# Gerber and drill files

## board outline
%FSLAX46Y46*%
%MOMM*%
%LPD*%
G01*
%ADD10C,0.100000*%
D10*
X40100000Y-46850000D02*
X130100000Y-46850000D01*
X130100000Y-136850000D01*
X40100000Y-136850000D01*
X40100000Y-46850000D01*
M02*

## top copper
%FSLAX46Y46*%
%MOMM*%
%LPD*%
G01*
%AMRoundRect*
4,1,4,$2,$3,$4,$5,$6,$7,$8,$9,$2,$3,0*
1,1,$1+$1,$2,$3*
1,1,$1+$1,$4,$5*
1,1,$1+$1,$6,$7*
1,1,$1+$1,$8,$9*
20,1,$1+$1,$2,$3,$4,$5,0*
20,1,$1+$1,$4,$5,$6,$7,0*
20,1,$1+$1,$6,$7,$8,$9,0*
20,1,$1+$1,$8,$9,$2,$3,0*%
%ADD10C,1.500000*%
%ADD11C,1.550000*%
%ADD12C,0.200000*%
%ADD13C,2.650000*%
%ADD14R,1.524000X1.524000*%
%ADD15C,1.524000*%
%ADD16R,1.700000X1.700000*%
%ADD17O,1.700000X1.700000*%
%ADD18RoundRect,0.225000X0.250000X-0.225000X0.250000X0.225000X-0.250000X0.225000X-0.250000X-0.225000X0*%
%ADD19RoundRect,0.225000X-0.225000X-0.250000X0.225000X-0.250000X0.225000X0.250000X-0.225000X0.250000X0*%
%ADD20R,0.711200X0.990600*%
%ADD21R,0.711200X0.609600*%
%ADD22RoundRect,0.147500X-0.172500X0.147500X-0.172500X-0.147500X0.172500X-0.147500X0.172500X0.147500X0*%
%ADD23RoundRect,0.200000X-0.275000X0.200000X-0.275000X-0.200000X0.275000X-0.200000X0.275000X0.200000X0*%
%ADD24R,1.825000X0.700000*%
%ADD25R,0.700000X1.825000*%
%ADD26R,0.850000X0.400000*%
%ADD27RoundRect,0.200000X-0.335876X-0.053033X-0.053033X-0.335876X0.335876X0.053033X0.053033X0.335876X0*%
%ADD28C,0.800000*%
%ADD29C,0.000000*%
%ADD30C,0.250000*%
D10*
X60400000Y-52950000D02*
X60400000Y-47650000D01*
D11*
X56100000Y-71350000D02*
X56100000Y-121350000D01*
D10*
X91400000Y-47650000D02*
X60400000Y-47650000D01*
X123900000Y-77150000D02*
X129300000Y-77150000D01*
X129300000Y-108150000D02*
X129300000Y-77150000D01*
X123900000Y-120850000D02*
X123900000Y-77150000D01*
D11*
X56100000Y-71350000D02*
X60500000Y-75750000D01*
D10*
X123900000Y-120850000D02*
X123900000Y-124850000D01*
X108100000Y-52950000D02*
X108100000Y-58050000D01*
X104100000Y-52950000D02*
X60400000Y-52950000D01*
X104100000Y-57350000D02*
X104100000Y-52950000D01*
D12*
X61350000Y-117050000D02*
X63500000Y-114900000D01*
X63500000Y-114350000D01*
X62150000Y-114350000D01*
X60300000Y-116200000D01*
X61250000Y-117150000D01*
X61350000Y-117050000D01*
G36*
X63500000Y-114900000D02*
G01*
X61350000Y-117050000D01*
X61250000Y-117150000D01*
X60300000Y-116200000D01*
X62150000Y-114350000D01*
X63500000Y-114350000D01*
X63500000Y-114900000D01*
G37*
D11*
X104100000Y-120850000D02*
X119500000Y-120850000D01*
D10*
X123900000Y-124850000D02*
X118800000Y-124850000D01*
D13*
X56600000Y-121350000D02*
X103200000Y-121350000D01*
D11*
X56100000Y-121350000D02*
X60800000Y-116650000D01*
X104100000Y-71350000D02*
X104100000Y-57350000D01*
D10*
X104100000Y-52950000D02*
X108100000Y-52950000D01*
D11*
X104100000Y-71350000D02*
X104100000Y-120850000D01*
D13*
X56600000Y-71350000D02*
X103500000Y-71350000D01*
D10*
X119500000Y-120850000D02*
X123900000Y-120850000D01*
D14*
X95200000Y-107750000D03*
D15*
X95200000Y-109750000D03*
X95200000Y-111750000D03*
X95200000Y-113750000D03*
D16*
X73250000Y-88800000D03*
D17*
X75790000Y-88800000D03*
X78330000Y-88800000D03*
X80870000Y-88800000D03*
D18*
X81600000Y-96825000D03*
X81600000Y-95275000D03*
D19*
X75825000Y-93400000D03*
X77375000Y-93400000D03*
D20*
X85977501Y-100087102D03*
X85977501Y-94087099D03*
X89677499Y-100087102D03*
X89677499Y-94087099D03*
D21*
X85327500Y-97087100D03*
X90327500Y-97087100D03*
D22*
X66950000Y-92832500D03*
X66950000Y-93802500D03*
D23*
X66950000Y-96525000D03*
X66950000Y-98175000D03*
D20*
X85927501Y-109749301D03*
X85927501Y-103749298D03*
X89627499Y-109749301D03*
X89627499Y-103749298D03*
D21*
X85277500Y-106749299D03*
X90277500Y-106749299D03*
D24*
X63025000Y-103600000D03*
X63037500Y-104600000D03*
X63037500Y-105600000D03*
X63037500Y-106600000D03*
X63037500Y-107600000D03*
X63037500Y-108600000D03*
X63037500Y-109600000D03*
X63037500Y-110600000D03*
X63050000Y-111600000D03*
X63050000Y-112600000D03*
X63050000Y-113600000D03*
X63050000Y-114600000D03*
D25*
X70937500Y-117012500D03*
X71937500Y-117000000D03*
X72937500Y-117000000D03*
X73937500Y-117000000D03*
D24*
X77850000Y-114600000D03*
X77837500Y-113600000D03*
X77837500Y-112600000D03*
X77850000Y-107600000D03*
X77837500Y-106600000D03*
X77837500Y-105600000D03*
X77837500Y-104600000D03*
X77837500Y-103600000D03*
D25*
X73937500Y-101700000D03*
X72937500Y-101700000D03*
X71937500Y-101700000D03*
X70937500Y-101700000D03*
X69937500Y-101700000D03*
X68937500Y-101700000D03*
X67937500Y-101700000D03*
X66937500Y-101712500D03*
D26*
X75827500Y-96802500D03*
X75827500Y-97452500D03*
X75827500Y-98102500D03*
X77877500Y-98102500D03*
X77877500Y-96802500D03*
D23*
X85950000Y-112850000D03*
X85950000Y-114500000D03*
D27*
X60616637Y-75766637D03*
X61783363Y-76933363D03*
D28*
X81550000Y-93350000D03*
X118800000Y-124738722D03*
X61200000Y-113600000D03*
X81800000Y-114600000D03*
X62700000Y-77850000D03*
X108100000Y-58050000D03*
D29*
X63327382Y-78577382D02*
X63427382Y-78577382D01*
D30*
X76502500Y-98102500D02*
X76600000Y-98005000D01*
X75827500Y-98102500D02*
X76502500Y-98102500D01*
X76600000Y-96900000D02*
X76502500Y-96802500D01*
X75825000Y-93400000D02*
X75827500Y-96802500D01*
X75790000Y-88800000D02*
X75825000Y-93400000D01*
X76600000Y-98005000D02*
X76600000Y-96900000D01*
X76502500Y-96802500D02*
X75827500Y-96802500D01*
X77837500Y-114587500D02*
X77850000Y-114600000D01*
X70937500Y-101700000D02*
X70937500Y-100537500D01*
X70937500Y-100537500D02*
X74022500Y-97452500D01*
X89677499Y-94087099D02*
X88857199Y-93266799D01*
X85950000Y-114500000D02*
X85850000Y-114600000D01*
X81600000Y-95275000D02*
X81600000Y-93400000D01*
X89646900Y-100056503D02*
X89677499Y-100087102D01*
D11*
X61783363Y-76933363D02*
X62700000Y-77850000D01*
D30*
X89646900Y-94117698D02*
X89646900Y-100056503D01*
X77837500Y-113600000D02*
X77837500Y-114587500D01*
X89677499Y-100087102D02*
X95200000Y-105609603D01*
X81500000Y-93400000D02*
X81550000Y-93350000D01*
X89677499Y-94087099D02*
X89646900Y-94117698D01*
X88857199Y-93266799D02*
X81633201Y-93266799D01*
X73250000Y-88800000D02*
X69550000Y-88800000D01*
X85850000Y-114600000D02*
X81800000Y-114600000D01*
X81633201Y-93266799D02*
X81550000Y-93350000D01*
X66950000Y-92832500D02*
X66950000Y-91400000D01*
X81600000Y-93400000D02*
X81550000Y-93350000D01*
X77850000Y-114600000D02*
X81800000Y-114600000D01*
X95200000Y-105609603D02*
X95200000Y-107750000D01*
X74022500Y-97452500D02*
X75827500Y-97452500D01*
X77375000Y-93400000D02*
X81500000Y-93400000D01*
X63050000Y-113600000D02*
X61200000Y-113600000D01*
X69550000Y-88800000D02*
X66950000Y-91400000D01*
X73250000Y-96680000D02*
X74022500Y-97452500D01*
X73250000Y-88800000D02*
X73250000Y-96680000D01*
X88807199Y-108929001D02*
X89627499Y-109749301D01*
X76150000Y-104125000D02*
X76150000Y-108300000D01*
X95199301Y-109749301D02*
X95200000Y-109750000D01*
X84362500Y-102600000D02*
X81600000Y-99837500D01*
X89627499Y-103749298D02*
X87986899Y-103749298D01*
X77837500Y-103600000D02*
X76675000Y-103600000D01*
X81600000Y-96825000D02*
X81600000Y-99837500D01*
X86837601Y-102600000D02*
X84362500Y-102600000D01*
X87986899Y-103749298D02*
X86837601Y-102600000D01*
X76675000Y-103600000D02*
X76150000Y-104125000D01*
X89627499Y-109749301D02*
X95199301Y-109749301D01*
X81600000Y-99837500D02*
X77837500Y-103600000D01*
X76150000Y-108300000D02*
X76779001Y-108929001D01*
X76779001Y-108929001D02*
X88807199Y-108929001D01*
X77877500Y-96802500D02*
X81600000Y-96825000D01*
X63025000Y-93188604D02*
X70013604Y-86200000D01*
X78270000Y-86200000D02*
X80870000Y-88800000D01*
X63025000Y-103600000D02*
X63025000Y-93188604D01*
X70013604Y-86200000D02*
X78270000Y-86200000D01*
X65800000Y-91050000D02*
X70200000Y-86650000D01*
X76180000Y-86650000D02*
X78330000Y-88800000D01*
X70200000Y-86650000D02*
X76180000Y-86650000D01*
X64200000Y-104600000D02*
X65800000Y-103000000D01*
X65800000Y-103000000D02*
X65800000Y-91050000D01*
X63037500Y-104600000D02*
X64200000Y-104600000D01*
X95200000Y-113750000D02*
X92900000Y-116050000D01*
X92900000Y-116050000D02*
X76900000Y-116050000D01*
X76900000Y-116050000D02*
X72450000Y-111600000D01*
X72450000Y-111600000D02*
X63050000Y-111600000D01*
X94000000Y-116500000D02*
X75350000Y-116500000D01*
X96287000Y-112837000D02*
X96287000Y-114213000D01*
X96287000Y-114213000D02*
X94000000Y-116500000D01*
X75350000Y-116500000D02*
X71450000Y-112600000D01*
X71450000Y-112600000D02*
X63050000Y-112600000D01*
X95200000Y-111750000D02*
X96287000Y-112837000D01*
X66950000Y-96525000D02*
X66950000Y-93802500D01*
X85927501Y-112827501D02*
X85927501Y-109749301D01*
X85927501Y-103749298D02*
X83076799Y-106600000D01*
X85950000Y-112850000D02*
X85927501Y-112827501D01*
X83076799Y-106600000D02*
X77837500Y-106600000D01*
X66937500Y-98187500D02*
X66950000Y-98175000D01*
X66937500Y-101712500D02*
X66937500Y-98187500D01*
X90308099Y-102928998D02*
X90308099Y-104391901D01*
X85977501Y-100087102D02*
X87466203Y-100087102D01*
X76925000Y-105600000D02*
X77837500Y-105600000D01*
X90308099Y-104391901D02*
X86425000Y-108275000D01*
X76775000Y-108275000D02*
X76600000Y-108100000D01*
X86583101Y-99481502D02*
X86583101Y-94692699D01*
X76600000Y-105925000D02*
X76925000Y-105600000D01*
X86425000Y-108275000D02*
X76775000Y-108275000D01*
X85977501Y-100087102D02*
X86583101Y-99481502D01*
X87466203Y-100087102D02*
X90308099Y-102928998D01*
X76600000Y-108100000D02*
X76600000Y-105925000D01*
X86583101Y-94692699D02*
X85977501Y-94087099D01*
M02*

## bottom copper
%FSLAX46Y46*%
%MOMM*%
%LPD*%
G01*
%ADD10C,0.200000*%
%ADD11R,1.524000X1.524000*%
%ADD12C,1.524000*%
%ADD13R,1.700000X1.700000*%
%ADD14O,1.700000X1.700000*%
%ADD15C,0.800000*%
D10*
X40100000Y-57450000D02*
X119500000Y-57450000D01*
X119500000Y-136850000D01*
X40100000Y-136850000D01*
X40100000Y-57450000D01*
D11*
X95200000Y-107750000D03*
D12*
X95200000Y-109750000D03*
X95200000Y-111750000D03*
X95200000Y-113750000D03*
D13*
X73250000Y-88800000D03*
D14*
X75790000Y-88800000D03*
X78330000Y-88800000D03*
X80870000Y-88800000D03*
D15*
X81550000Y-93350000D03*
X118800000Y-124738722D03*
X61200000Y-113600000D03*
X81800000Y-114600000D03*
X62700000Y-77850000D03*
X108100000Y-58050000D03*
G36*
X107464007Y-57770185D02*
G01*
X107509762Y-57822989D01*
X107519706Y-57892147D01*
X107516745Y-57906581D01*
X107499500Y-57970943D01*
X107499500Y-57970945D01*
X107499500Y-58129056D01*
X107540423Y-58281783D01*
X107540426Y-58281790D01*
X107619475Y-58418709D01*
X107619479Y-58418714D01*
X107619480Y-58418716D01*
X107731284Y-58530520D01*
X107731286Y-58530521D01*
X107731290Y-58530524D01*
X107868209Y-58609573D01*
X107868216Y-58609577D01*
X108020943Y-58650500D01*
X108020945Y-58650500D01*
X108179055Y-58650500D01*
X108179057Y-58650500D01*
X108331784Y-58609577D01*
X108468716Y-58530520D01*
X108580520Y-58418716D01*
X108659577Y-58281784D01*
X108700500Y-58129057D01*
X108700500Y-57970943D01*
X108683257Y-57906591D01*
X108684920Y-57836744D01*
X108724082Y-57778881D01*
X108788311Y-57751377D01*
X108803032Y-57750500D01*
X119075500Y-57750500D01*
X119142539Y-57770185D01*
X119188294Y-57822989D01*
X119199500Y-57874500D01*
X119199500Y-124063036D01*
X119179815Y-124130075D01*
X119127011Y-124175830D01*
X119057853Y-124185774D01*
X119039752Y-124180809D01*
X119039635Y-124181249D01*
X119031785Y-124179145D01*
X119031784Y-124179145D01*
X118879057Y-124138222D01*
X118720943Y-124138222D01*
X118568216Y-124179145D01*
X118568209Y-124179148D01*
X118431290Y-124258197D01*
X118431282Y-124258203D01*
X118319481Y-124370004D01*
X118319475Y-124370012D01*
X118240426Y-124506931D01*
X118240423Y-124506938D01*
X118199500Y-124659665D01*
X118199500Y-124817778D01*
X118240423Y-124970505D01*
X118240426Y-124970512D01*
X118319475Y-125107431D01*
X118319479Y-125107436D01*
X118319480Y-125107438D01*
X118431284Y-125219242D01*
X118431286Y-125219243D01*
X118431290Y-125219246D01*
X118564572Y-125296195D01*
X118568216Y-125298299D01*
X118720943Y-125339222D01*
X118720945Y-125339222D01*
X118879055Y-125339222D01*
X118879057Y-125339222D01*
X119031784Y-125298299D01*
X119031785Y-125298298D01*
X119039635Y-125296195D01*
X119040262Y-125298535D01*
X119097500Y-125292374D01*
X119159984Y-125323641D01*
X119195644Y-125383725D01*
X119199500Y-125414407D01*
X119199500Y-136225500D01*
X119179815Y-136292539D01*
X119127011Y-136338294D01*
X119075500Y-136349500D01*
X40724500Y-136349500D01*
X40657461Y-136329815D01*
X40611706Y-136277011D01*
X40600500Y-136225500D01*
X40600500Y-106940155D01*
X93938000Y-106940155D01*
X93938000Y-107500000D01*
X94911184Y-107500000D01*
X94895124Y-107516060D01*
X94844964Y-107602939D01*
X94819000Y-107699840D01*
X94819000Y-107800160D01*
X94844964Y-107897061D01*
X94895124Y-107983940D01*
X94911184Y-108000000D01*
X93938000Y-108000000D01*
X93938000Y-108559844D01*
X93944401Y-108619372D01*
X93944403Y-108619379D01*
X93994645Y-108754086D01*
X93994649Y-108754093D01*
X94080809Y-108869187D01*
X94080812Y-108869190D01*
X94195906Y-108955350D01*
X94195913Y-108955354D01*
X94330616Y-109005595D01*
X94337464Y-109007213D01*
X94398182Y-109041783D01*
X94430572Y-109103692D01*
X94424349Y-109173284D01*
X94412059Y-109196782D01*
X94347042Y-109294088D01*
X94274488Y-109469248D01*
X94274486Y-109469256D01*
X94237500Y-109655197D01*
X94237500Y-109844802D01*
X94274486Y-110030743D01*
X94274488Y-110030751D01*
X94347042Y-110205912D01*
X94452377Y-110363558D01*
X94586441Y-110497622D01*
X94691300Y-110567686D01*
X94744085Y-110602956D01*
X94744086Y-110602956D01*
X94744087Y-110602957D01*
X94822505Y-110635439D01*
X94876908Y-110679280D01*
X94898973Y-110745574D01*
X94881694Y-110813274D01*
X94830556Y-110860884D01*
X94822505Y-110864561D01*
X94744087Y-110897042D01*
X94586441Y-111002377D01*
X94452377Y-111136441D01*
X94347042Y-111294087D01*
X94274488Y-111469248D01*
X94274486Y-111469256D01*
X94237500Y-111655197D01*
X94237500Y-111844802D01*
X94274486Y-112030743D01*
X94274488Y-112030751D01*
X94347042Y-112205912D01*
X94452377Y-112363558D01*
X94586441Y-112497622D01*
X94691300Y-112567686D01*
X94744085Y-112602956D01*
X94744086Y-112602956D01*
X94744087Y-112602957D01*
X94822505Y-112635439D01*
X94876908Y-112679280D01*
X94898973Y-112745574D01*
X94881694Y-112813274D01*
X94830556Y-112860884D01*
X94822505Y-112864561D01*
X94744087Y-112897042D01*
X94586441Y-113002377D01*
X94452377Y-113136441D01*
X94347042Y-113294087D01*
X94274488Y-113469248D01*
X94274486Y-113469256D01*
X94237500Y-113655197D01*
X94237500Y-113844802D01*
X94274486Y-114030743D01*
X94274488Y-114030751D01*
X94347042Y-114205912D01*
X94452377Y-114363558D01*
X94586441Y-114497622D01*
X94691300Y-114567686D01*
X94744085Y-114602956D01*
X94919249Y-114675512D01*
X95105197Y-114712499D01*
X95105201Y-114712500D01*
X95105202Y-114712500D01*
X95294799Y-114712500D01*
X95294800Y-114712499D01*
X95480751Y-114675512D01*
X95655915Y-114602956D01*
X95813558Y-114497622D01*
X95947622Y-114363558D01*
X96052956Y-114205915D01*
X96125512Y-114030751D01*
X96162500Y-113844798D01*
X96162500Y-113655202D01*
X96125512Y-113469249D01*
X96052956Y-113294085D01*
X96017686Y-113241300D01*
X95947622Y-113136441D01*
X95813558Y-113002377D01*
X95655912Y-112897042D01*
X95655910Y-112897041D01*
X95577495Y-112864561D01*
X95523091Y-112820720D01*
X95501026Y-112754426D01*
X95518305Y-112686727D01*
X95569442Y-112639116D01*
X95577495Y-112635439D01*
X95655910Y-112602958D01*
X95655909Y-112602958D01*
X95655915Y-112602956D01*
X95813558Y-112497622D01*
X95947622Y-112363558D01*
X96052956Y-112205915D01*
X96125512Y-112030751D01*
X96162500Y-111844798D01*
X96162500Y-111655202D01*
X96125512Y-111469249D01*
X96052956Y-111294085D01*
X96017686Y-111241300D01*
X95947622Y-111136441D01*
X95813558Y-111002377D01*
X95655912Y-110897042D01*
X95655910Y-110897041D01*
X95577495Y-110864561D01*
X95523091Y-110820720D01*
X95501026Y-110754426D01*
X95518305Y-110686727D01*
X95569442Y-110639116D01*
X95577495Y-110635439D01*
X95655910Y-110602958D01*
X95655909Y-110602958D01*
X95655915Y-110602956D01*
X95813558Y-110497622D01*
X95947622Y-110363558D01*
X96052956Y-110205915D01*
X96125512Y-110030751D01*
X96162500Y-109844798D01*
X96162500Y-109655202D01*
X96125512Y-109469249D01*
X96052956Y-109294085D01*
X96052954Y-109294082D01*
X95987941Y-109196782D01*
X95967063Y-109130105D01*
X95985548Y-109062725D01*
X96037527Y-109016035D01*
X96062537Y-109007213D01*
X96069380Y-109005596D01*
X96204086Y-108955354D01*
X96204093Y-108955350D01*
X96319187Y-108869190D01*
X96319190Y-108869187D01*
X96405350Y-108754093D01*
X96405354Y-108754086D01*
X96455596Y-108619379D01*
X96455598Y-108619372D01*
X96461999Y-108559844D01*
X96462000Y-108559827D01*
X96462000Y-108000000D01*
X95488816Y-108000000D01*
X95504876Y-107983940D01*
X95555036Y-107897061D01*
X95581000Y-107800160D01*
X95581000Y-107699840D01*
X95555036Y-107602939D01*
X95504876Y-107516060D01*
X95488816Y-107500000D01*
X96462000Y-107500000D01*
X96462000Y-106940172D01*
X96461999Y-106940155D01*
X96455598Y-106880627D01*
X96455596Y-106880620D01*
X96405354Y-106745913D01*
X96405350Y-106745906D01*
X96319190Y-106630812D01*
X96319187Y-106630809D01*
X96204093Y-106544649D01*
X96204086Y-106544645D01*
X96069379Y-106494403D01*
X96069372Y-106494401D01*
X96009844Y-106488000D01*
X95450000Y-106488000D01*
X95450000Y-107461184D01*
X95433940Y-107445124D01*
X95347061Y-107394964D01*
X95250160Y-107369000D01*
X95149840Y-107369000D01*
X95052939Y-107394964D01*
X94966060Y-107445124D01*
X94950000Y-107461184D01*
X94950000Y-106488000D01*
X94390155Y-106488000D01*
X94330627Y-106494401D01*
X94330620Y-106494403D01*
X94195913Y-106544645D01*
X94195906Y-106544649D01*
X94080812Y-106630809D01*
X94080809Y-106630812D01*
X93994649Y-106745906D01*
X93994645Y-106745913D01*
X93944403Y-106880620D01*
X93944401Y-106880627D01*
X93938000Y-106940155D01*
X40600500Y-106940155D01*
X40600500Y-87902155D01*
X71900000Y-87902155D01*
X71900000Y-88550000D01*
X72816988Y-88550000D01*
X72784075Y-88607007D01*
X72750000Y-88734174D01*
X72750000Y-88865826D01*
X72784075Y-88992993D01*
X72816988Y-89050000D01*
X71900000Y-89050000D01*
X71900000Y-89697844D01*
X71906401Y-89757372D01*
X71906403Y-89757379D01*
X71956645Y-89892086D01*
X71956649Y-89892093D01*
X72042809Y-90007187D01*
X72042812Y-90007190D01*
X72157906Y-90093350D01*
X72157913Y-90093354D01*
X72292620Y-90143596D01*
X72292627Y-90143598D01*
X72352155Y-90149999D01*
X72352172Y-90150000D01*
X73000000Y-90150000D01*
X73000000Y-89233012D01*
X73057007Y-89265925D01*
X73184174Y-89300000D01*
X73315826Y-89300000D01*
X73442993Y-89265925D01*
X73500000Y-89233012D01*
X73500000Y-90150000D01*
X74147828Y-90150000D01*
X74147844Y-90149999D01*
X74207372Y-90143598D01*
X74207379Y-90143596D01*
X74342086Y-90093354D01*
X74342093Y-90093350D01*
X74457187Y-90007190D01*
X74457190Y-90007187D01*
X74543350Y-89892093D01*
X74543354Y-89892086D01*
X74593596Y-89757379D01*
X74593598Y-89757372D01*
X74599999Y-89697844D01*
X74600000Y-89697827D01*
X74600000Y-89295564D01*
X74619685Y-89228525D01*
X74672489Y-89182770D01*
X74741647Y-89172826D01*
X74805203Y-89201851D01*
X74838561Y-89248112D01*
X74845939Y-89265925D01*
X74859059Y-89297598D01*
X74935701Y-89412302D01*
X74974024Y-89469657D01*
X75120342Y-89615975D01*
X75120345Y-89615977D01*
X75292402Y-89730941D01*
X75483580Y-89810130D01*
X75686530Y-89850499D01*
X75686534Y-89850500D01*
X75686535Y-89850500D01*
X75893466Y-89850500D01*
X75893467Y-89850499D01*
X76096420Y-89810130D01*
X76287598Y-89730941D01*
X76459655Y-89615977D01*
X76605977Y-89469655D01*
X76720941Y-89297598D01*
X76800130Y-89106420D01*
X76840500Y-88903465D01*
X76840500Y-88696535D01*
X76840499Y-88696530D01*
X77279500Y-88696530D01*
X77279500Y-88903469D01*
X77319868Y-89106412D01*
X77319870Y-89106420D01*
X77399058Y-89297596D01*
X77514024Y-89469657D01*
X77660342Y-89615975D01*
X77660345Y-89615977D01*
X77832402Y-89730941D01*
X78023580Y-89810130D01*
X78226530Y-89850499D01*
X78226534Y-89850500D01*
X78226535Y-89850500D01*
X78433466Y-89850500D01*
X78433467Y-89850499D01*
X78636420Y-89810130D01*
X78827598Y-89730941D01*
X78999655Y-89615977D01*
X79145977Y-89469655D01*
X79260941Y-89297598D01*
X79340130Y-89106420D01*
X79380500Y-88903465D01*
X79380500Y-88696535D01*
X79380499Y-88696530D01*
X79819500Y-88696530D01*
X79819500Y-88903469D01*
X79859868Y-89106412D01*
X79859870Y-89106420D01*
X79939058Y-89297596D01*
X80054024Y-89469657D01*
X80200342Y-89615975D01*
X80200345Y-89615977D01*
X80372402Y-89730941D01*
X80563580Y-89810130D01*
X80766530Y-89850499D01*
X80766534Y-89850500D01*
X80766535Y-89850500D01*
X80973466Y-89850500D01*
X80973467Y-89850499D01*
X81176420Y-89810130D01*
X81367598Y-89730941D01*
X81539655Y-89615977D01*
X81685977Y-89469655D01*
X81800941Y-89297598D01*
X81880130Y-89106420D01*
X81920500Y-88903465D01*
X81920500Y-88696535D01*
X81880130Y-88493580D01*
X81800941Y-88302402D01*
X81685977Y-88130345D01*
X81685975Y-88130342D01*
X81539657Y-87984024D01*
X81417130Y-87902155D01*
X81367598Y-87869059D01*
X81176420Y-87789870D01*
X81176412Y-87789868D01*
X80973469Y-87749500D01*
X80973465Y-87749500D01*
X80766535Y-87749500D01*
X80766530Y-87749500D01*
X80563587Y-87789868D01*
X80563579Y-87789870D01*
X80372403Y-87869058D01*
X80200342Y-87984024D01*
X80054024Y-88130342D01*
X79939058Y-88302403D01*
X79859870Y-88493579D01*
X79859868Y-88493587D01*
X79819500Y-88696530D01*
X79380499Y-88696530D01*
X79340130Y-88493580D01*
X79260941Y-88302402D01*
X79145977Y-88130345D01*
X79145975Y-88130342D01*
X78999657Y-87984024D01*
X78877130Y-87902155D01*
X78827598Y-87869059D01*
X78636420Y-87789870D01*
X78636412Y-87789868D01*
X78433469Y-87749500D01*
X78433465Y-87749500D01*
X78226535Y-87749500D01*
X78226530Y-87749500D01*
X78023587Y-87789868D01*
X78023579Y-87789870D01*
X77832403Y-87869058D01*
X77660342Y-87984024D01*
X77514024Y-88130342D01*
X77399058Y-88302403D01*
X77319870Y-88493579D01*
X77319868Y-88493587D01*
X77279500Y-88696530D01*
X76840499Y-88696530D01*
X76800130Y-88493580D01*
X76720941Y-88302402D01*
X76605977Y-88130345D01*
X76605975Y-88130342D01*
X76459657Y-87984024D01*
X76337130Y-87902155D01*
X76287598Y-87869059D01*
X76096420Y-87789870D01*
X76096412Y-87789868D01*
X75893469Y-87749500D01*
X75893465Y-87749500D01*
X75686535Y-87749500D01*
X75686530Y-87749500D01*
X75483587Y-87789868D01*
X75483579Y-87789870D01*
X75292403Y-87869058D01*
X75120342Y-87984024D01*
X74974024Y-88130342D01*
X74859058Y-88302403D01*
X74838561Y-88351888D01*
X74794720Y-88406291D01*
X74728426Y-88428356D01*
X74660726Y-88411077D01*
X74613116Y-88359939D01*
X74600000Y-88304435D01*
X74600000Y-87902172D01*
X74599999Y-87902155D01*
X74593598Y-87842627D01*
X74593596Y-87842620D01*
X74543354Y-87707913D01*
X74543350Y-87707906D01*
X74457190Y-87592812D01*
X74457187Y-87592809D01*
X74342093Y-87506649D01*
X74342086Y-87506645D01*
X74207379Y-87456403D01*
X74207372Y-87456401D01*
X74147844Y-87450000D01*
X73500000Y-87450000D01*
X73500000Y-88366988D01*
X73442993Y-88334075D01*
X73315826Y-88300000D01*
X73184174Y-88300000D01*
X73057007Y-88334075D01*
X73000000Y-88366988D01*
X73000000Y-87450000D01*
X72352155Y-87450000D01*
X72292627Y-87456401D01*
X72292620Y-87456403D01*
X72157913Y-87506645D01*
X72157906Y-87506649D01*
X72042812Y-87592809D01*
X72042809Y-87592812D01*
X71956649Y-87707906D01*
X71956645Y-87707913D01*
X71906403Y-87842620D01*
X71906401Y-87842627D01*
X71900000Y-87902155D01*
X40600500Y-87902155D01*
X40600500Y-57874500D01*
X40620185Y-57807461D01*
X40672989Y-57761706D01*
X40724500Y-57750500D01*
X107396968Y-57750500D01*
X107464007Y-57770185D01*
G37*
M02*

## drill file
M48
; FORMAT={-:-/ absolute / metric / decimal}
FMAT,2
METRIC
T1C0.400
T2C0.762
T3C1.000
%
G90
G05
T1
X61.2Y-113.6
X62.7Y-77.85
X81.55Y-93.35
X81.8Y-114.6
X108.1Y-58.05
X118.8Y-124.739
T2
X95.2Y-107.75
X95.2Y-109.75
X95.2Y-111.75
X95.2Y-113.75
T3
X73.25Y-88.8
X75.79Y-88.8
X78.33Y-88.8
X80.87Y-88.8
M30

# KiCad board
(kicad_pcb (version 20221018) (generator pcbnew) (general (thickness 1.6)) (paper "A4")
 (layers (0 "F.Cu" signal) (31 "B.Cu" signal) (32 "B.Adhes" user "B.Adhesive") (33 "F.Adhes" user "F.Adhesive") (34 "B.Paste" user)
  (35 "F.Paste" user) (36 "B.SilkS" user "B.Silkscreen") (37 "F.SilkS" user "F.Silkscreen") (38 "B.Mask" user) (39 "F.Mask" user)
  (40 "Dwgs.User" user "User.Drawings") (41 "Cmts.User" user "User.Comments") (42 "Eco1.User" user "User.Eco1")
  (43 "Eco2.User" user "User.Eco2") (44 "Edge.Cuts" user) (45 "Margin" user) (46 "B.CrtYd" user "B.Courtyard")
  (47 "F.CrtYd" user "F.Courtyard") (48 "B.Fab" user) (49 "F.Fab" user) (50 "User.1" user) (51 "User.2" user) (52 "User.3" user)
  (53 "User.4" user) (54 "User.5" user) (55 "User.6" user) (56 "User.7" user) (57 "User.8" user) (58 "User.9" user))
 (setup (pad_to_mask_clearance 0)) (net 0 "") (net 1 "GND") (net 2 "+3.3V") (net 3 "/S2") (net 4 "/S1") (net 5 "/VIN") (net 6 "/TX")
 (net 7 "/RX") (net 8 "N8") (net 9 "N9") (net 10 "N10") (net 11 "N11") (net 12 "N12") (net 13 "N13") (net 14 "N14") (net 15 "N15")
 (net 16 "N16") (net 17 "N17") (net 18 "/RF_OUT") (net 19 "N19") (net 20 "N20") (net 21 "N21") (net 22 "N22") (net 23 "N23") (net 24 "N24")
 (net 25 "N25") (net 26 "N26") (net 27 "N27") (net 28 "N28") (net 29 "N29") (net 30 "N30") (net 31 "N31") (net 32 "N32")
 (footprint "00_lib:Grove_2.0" (layer "F.Cu") (at 95.05 110.75)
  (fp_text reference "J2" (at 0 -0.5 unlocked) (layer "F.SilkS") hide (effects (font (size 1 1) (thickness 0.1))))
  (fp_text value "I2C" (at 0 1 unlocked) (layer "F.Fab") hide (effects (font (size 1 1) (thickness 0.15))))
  (pad "1" thru_hole rect (at 0.15 -3) (size 1.524 1.524) (drill 0.762) (layers "*.Cu" "*.Mask") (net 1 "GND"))
  (pad "2" thru_hole circle (at 0.15 -1) (size 1.524 1.524) (drill 0.762) (layers "*.Cu" "*.Mask") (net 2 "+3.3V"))
  (pad "3" thru_hole circle (at 0.15 1) (size 1.524 1.524) (drill 0.762) (layers "*.Cu" "*.Mask") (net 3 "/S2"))
  (pad "4" thru_hole circle (at 0.15 3) (size 1.524 1.524) (drill 0.762) (layers "*.Cu" "*.Mask") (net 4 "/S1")))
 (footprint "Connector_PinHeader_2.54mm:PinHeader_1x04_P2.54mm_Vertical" (layer "F.Cu") (at 73.25 88.8 90)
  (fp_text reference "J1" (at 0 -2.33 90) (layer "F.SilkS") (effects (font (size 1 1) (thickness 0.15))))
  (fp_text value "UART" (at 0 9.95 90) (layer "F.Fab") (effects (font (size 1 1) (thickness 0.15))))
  (pad "1" thru_hole rect (at 0 0 90) (size 1.7 1.7) (drill 1) (layers "*.Cu" "*.Mask") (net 1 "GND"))
  (pad "2" thru_hole oval (at 0 2.54 90) (size 1.7 1.7) (drill 1) (layers "*.Cu" "*.Mask") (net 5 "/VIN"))
  (pad "3" thru_hole oval (at 0 5.08 90) (size 1.7 1.7) (drill 1) (layers "*.Cu" "*.Mask") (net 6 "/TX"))
  (pad "4" thru_hole oval (at 0 7.62 90) (size 1.7 1.7) (drill 1) (layers "*.Cu" "*.Mask") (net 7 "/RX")))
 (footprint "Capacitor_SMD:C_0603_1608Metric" (layer "F.Cu") (at 81.6 96.05 90)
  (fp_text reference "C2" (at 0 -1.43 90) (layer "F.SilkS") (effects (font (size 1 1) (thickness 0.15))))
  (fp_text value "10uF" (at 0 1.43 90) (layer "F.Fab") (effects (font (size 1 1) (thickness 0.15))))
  (pad "1" smd roundrect (at -0.775 0 90) (size 0.9 0.95) (layers "F.Cu" "F.Paste" "F.Mask") (roundrect_rratio 0.25) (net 2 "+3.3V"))
  (pad "2" smd roundrect (at 0.775 0 90) (size 0.9 0.95) (layers "F.Cu" "F.Paste" "F.Mask") (roundrect_rratio 0.25) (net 1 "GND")))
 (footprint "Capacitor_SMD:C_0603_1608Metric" (layer "F.Cu") (at 76.6 93.4)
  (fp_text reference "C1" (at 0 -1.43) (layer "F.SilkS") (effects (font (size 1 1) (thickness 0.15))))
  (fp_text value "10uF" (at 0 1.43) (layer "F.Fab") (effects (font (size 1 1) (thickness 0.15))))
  (pad "1" smd roundrect (at -0.775 0) (size 0.9 0.95) (layers "F.Cu" "F.Paste" "F.Mask") (roundrect_rratio 0.25) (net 5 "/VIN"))
  (pad "2" smd roundrect (at 0.775 0) (size 0.9 0.95) (layers "F.Cu" "F.Paste" "F.Mask") (roundrect_rratio 0.25) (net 1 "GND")))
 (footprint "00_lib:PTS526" (layer "F.Cu") (at 87.7363 97.037801 90)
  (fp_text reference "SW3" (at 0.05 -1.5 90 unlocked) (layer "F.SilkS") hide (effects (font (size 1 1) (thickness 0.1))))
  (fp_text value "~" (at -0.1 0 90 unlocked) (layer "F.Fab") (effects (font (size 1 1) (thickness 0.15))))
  (pad "1" smd rect (at -3.049301 -1.758799 90) (size 0.9906 0.7112) (layers "F.Cu" "F.Paste" "F.Mask") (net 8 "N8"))
  (pad "2" smd rect (at 2.950702 -1.758799 90) (size 0.9906 0.7112) (layers "F.Cu" "F.Paste" "F.Mask") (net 8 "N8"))
  (pad "3" smd rect (at -3.049301 1.941199 90) (size 0.9906 0.7112) (layers "F.Cu" "F.Paste" "F.Mask") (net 1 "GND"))
  (pad "4" smd rect (at 2.950702 1.941199 90) (size 0.9906 0.7112) (layers "F.Cu" "F.Paste" "F.Mask") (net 1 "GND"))
  (pad "5" smd rect (at -0.049299 -2.4088 180) (size 0.7112 0.6096) (layers "F.Cu" "F.Paste" "F.Mask"))
  (pad "6" smd rect (at -0.049299 2.5912 180) (size 0.7112 0.6096) (layers "F.Cu" "F.Paste" "F.Mask")))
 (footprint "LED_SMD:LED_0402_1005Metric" (layer "F.Cu") (at 66.95 93.3175 -90)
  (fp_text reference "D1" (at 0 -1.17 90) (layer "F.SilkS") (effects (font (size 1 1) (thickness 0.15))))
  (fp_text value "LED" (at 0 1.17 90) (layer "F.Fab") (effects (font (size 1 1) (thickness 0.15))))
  (pad "1" smd roundrect (at -0.485 0 270) (size 0.59 0.64) (layers "F.Cu" "F.Paste" "F.Mask") (roundrect_rratio 0.25) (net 1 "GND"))
  (pad "2" smd roundrect (at 0.485 0 270) (size 0.59 0.64) (layers "F.Cu" "F.Paste" "F.Mask") (roundrect_rratio 0.25) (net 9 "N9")))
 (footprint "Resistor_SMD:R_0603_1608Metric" (layer "F.Cu") (at 66.95 97.35 -90)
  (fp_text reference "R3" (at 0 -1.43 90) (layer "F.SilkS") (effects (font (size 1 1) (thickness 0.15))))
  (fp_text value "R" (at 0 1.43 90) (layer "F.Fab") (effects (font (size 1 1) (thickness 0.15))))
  (pad "1" smd roundrect (at -0.825 0 270) (size 0.8 0.95) (layers "F.Cu" "F.Paste" "F.Mask") (roundrect_rratio 0.25) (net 9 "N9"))
  (pad "2" smd roundrect (at 0.825 0 270) (size 0.8 0.95) (layers "F.Cu" "F.Paste" "F.Mask") (roundrect_rratio 0.25) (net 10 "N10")))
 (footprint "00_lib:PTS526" (layer "F.Cu") (at 87.6863 106.7 90)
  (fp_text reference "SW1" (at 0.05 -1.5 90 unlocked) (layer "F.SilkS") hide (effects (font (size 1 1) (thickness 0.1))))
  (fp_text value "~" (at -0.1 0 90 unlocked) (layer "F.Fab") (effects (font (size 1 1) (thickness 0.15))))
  (pad "1" smd rect (at -3.049301 -1.758799 90) (size 0.9906 0.7112) (layers "F.Cu" "F.Paste" "F.Mask") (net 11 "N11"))
  (pad "2" smd rect (at 2.950702 -1.758799 90) (size 0.9906 0.7112) (layers "F.Cu" "F.Paste" "F.Mask") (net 11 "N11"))
  (pad "3" smd rect (at -3.049301 1.941199 90) (size 0.9906 0.7112) (layers "F.Cu" "F.Paste" "F.Mask") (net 2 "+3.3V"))
  (pad "4" smd rect (at 2.950702 1.941199 90) (size 0.9906 0.7112) (layers "F.Cu" "F.Paste" "F.Mask") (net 2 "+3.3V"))
  (pad "5" smd rect (at -0.049299 -2.4088 180) (size 0.7112 0.6096) (layers "F.Cu" "F.Paste" "F.Mask"))
  (pad "6" smd rect (at -0.049299 2.5912 180) (size 0.7112 0.6096) (layers "F.Cu" "F.Paste" "F.Mask")))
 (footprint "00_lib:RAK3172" (layer "F.Cu") (at 70.4875 109.35 90)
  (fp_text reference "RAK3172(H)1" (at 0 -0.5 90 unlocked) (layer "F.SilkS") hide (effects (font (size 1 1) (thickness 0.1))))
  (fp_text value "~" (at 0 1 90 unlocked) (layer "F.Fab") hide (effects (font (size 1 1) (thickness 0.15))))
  (pad "1" smd rect (at 5.75 -7.4625 180) (size 1.825 0.7) (layers "F.Cu" "F.Paste" "F.Mask") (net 7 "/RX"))
  (pad "2" smd rect (at 4.75 -7.45 180) (size 1.825 0.7) (layers "F.Cu" "F.Paste" "F.Mask") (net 6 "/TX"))
  (pad "3" smd rect (at 3.75 -7.45 180) (size 1.825 0.7) (layers "F.Cu" "F.Paste" "F.Mask") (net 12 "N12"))
  (pad "4" smd rect (at 2.75 -7.45 180) (size 1.825 0.7) (layers "F.Cu" "F.Paste" "F.Mask") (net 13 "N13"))
  (pad "5" smd rect (at 1.75 -7.45 180) (size 1.825 0.7) (layers "F.Cu" "F.Paste" "F.Mask") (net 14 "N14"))
  (pad "6" smd rect (at 0.75 -7.45 180) (size 1.825 0.7) (layers "F.Cu" "F.Paste" "F.Mask") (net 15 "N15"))
  (pad "7" smd rect (at -0.25 -7.45 180) (size 1.825 0.7) (layers "F.Cu" "F.Paste" "F.Mask") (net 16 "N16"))
  (pad "8" smd rect (at -1.25 -7.45 180) (size 1.825 0.7) (layers "F.Cu" "F.Paste" "F.Mask") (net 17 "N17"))
  (pad "9" smd rect (at -2.25 -7.4375 180) (size 1.825 0.7) (layers "F.Cu" "F.Paste" "F.Mask") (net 4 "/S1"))
  (pad "10" smd rect (at -3.25 -7.4375 180) (size 1.825 0.7) (layers "F.Cu" "F.Paste" "F.Mask") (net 3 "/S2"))
  (pad "11" smd rect (at -4.25 -7.4375 180) (size 1.825 0.7) (layers "F.Cu" "F.Paste" "F.Mask") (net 1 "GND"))
  (pad "12" smd rect (at -5.25 -7.4375 180) (size 1.825 0.7) (layers "F.Cu" "F.Paste" "F.Mask") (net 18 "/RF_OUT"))
  (pad "13" smd rect (at -7.6625 0.45 270) (size 1.825 0.7) (layers "F.Cu" "F.Paste" "F.Mask") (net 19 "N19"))
  (pad "14" smd rect (at -7.65 1.45 270) (size 1.825 0.7) (layers "F.Cu" "F.Paste" "F.Mask") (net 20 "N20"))
  (pad "15" smd rect (at -7.65 2.45 270) (size 1.825 0.7) (layers "F.Cu" "F.Paste" "F.Mask") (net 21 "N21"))
  (pad "16" smd rect (at -7.65 3.45 270) (size 1.825 0.7) (layers "F.Cu" "F.Paste" "F.Mask") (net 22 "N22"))
  (pad "17" smd rect (at -5.25 7.3625) (size 1.825 0.7) (layers "F.Cu" "F.Paste" "F.Mask") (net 1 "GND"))
  (pad "18" smd rect (at -4.25 7.35) (size 1.825 0.7) (layers "F.Cu" "F.Paste" "F.Mask") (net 1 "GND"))
  (pad "19" smd rect (at -3.25 7.35) (size 1.825 0.7) (layers "F.Cu" "F.Paste" "F.Mask") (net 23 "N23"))
  (pad "20" smd rect (at 1.75 7.3625) (size 1.825 0.7) (layers "F.Cu" "F.Paste" "F.Mask") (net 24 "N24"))
  (pad "21" smd rect (at 2.75 7.35) (size 1.825 0.7) (layers "F.Cu" "F.Paste" "F.Mask") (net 11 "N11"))
  (pad "22" smd rect (at 3.75 7.35) (size 1.825 0.7) (layers "F.Cu" "F.Paste" "F.Mask") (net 8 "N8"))
  (pad "23" smd rect (at 4.75 7.35) (size 1.825 0.7) (layers "F.Cu" "F.Paste" "F.Mask") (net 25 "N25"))
  (pad "24" smd rect (at 5.75 7.35) (size 1.825 0.7) (layers "F.Cu" "F.Paste" "F.Mask") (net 2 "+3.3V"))
  (pad "25" smd rect (at 7.65 3.45 270) (size 1.825 0.7) (layers "F.Cu" "F.Paste" "F.Mask") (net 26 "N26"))
  (pad "26" smd rect (at 7.65 2.45 270) (size 1.825 0.7) (layers "F.Cu" "F.Paste" "F.Mask") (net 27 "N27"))
  (pad "27" smd rect (at 7.65 1.45 270) (size 1.825 0.7) (layers "F.Cu" "F.Paste" "F.Mask") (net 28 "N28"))
  (pad "28" smd rect (at 7.65 0.45 270) (size 1.825 0.7) (layers "F.Cu" "F.Paste" "F.Mask") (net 1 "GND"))
  (pad "29" smd rect (at 7.65 -0.55 270) (size 1.825 0.7) (layers "F.Cu" "F.Paste" "F.Mask") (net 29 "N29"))
  (pad "30" smd rect (at 7.65 -1.55 270) (size 1.825 0.7) (layers "F.Cu" "F.Paste" "F.Mask") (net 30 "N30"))
  (pad "31" smd rect (at 7.65 -2.55 270) (size 1.825 0.7) (layers "F.Cu" "F.Paste" "F.Mask") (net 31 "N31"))
  (pad "32" smd rect (at 7.6375 -3.55 270) (size 1.825 0.7) (layers "F.Cu" "F.Paste" "F.Mask") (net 10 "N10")))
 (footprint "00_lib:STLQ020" (layer "F.Cu") (at 76.9025 97.5025)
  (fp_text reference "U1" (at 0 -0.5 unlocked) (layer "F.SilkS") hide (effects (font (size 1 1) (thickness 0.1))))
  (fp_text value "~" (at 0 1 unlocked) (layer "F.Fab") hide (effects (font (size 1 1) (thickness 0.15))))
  (pad "1" smd rect (at -1.075 -0.7) (size 0.85 0.4) (layers "F.Cu" "F.Paste" "F.Mask") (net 5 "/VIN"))
  (pad "2" smd rect (at -1.075 -0.05) (size 0.85 0.4) (layers "F.Cu" "F.Paste" "F.Mask") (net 1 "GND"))
  (pad "3" smd rect (at -1.075 0.6) (size 0.85 0.4) (layers "F.Cu" "F.Paste" "F.Mask") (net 5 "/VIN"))
  (pad "4" smd rect (at 0.975 0.6) (size 0.85 0.4) (layers "F.Cu" "F.Paste" "F.Mask") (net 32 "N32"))
  (pad "5" smd rect (at 0.975 -0.7) (size 0.85 0.4) (layers "F.Cu" "F.Paste" "F.Mask") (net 2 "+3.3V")))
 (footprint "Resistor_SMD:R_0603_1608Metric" (layer "F.Cu") (at 85.95 113.675 -90)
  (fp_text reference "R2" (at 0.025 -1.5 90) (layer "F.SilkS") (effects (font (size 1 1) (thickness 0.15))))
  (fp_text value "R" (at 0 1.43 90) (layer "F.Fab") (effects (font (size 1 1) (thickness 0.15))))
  (pad "1" smd roundrect (at -0.825 0 270) (size 0.8 0.95) (layers "F.Cu" "F.Paste" "F.Mask") (roundrect_rratio 0.25) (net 11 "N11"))
  (pad "2" smd roundrect (at 0.825 0 270) (size 0.8 0.95) (layers "F.Cu" "F.Paste" "F.Mask") (roundrect_rratio 0.25) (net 1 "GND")))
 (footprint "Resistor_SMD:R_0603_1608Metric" (layer "F.Cu") (at 61.2 76.35 -45)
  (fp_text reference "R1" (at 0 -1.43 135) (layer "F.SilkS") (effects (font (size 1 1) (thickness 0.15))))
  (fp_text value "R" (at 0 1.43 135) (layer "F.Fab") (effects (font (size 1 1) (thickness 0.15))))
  (pad "1" smd roundrect (at -0.825 0 315) (size 0.8 0.95) (layers "F.Cu" "F.Paste" "F.Mask") (roundrect_rratio 0.25) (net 18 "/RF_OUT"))
  (pad "2" smd roundrect (at 0.825 0 315) (size 0.8 0.95) (layers "F.Cu" "F.Paste" "F.Mask") (roundrect_rratio 0.25) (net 1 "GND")))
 (gr_line (start 60.4 52.95) (end 60.4 47.65) (stroke (width 1.5) (type default)) (layer "F.Cu"))
 (gr_line (start 56.1 71.35) (end 56.1 121.35) (stroke (width 1.55) (type default)) (layer "F.Cu"))
 (gr_line (start 91.4 47.65) (end 60.4 47.65) (stroke (width 1.5) (type default)) (layer "F.Cu"))
 (gr_line (start 123.9 77.15) (end 129.3 77.15) (stroke (width 1.5) (type default)) (layer "F.Cu"))
 (gr_line (start 129.3 108.15) (end 129.3 77.15) (stroke (width 1.5) (type default)) (layer "F.Cu"))
 (gr_line (start 123.9 120.85) (end 123.9 77.15) (stroke (width 1.5) (type default)) (layer "F.Cu"))
 (gr_line (start 56.1 71.35) (end 60.5 75.75) (stroke (width 1.55) (type default)) (layer "F.Cu"))
 (gr_line (start 123.9 120.85) (end 123.9 124.85) (stroke (width 1.5) (type default)) (layer "F.Cu"))
 (gr_line (start 108.1 52.95) (end 108.1 58.05) (stroke (width 1.5) (type default)) (layer "F.Cu"))
 (gr_line (start 104.1 52.95) (end 60.4 52.95) (stroke (width 1.5) (type default)) (layer "F.Cu"))
 (gr_line (start 104.1 57.35) (end 104.1 52.95) (stroke (width 1.5) (type default)) (layer "F.Cu"))
 (gr_poly
  (pts (xy 61.35 117.05) (xy 63.5 114.9) (xy 63.5 114.35) (xy 62.15 114.35) (xy 60.3 116.2) (xy 61.25 117.15))
  (stroke (width 0.2) (type solid)) (fill solid) (layer "F.Cu"))
 (gr_line (start 104.1 120.85) (end 119.5 120.85) (stroke (width 1.55) (type default)) (layer "F.Cu"))
 (gr_line (start 123.9 124.85) (end 118.8 124.85) (stroke (width 1.5) (type default)) (layer "F.Cu"))
 (gr_line (start 56.6 121.35) (end 103.2 121.35) (stroke (width 2.65) (type default)) (layer "F.Cu"))
 (gr_line (start 56.1 121.35) (end 60.8 116.65) (stroke (width 1.55) (type default)) (layer "F.Cu"))
 (gr_line (start 104.1 71.35) (end 104.1 57.35) (stroke (width 1.55) (type default)) (layer "F.Cu"))
 (gr_line (start 104.1 52.95) (end 108.1 52.95) (stroke (width 1.5) (type default)) (layer "F.Cu"))
 (gr_line (start 104.1 71.35) (end 104.1 120.85) (stroke (width 1.55) (type default)) (layer "F.Cu"))
 (gr_line (start 56.6 71.35) (end 103.5 71.35) (stroke (width 2.65) (type default)) (layer "F.Cu"))
 (gr_line (start 119.5 120.85) (end 123.9 120.85) (stroke (width 1.5) (type default)) (layer "F.Cu"))
 (gr_rect (start 40.1 57.45) (end 119.5 136.85) (stroke (width 0.2) (type default)) (fill none) (layer "B.Cu"))
 (gr_rect (start 40.1 46.85) (end 130.1 136.85) (stroke (width 0.1) (type default)) (fill none) (layer "Edge.Cuts"))
 (segment (start 63.327382 78.577382) (end 63.427382 78.577382) (width 0) (layer "F.Cu") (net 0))
 (segment (start 76.5025 98.1025) (end 76.6 98.005) (width 0.25) (layer "F.Cu") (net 5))
 (segment (start 75.8275 98.1025) (end 76.5025 98.1025) (width 0.25) (layer "F.Cu") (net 5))
 (segment (start 76.6 96.9) (end 76.5025 96.8025) (width 0.25) (layer "F.Cu") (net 5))
 (segment (start 75.825 93.4) (end 75.8275 96.8025) (width 0.25) (layer "F.Cu") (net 5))
 (segment (start 75.79 88.8) (end 75.825 93.4) (width 0.25) (layer "F.Cu") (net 5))
 (segment (start 76.6 98.005) (end 76.6 96.9) (width 0.25) (layer "F.Cu") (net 5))
 (segment (start 76.5025 96.8025) (end 75.8275 96.8025) (width 0.25) (layer "F.Cu") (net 5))
 (segment (start 77.8375 114.5875) (end 77.85 114.6) (width 0.25) (layer "F.Cu") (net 1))
 (segment (start 70.9375 101.7) (end 70.9375 100.5375) (width 0.25) (layer "F.Cu") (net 1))
 (segment (start 70.9375 100.5375) (end 74.0225 97.4525) (width 0.25) (layer "F.Cu") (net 1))
 (segment (start 89.677499 94.087099) (end 88.857199 93.266799) (width 0.25) (layer "F.Cu") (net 1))
 (segment (start 85.95 114.5) (end 85.85 114.6) (width 0.25) (layer "F.Cu") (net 1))
 (segment (start 81.6 95.275) (end 81.6 93.4) (width 0.25) (layer "F.Cu") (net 1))
 (segment (start 89.6469 100.056503) (end 89.677499 100.087102) (width 0.25) (layer "F.Cu") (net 1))
 (segment (start 61.783363 76.933363) (end 62.7 77.85) (width 1.55) (layer "F.Cu") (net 1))
 (segment (start 89.6469 94.117698) (end 89.6469 100.056503) (width 0.25) (layer "F.Cu") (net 1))
 (segment (start 77.8375 113.6) (end 77.8375 114.5875) (width 0.25) (layer "F.Cu") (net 1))
 (segment (start 89.677499 100.087102) (end 95.2 105.609603) (width 0.25) (layer "F.Cu") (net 1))
 (segment (start 81.5 93.4) (end 81.55 93.35) (width 0.25) (layer "F.Cu") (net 1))
 (segment (start 89.677499 94.087099) (end 89.6469 94.117698) (width 0.25) (layer "F.Cu") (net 1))
 (segment (start 88.857199 93.266799) (end 81.633201 93.266799) (width 0.25) (layer "F.Cu") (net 1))
 (segment (start 73.25 88.8) (end 69.55 88.8) (width 0.25) (layer "F.Cu") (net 1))
 (segment (start 85.85 114.6) (end 81.8 114.6) (width 0.25) (layer "F.Cu") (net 1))
 (segment (start 81.633201 93.266799) (end 81.55 93.35) (width 0.25) (layer "F.Cu") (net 1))
 (segment (start 66.95 92.8325) (end 66.95 91.4) (width 0.25) (layer "F.Cu") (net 1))
 (segment (start 81.6 93.4) (end 81.55 93.35) (width 0.25) (layer "F.Cu") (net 1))
 (segment (start 77.85 114.6) (end 81.8 114.6) (width 0.25) (layer "F.Cu") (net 1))
 (segment (start 95.2 105.609603) (end 95.2 107.75) (width 0.25) (layer "F.Cu") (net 1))
 (segment (start 74.0225 97.4525) (end 75.8275 97.4525) (width 0.25) (layer "F.Cu") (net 1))
 (segment (start 77.375 93.4) (end 81.5 93.4) (width 0.25) (layer "F.Cu") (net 1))
 (segment (start 63.05 113.6) (end 61.2 113.6) (width 0.25) (layer "F.Cu") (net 1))
 (segment (start 69.55 88.8) (end 66.95 91.4) (width 0.25) (layer "F.Cu") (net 1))
 (segment (start 73.25 96.68) (end 74.0225 97.4525) (width 0.25) (layer "F.Cu") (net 1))
 (segment (start 73.25 88.8) (end 73.25 96.68) (width 0.25) (layer "F.Cu") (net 1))
 (via (at 81.55 93.35) (size 0.8) (drill 0.4) (layers "F.Cu" "B.Cu") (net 1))
 (via (at 118.8 124.738722) (size 0.8) (drill 0.4) (layers "F.Cu" "B.Cu") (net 1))
 (via (at 61.2 113.6) (size 0.8) (drill 0.4) (layers "F.Cu" "B.Cu") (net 1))
 (via (at 81.8 114.6) (size 0.8) (drill 0.4) (layers "F.Cu" "B.Cu") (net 1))
 (via (at 62.7 77.85) (size 0.8) (drill 0.4) (layers "F.Cu" "B.Cu") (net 1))
 (via (at 108.1 58.05) (size 0.8) (drill 0.4) (layers "F.Cu" "B.Cu") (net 1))
 (segment (start 88.807199 108.929001) (end 89.627499 109.749301) (width 0.25) (layer "F.Cu") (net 2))
 (segment (start 76.15 104.125) (end 76.15 108.3) (width 0.25) (layer "F.Cu") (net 2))
 (segment (start 95.199301 109.749301) (end 95.2 109.75) (width 0.25) (layer "F.Cu") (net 2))
 (segment (start 84.3625 102.6) (end 81.6 99.8375) (width 0.25) (layer "F.Cu") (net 2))
 (segment (start 89.627499 103.749298) (end 87.986899 103.749298) (width 0.25) (layer "F.Cu") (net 2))
 (segment (start 77.8375 103.6) (end 76.675 103.6) (width 0.25) (layer "F.Cu") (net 2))
 (segment (start 81.6 96.825) (end 81.6 99.8375) (width 0.25) (layer "F.Cu") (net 2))
 (segment (start 86.837601 102.6) (end 84.3625 102.6) (width 0.25) (layer "F.Cu") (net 2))
 (segment (start 87.986899 103.749298) (end 86.837601 102.6) (width 0.25) (layer "F.Cu") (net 2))
 (segment (start 76.675 103.6) (end 76.15 104.125) (width 0.25) (layer "F.Cu") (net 2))
 (segment (start 89.627499 109.749301) (end 95.199301 109.749301) (width 0.25) (layer "F.Cu") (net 2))
 (segment (start 81.6 99.8375) (end 77.8375 103.6) (width 0.25) (layer "F.Cu") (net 2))
 (segment (start 76.15 108.3) (end 76.779001 108.929001) (width 0.25) (layer "F.Cu") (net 2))
 (segment (start 76.779001 108.929001) (end 88.807199 108.929001) (width 0.25) (layer "F.Cu") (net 2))
 (segment (start 77.8775 96.8025) (end 81.6 96.825) (width 0.25) (layer "F.Cu") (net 2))
 (segment (start 63.025 93.188604) (end 70.013604 86.2) (width 0.25) (layer "F.Cu") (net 7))
 (segment (start 78.27 86.2) (end 80.87 88.8) (width 0.25) (layer "F.Cu") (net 7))
 (segment (start 63.025 103.6) (end 63.025 93.188604) (width 0.25) (layer "F.Cu") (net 7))
 (segment (start 70.013604 86.2) (end 78.27 86.2) (width 0.25) (layer "F.Cu") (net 7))
 (segment (start 65.8 91.05) (end 70.2 86.65) (width 0.25) (layer "F.Cu") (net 6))
 (segment (start 76.18 86.65) (end 78.33 88.8) (width 0.25) (layer "F.Cu") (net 6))
 (segment (start 70.2 86.65) (end 76.18 86.65) (width 0.25) (layer "F.Cu") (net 6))
 (segment (start 64.2 104.6) (end 65.8 103) (width 0.25) (layer "F.Cu") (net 6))
 (segment (start 65.8 103) (end 65.8 91.05) (width 0.25) (layer "F.Cu") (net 6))
 (segment (start 63.0375 104.6) (end 64.2 104.6) (width 0.25) (layer "F.Cu") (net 6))
 (segment (start 95.2 113.75) (end 92.9 116.05) (width 0.25) (layer "F.Cu") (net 4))
 (segment (start 92.9 116.05) (end 76.9 116.05) (width 0.25) (layer "F.Cu") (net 4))
 (segment (start 76.9 116.05) (end 72.45 111.6) (width 0.25) (layer "F.Cu") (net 4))
 (segment (start 72.45 111.6) (end 63.05 111.6) (width 0.25) (layer "F.Cu") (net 4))
 (segment (start 94 116.5) (end 75.35 116.5) (width 0.25) (layer "F.Cu") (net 3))
 (segment (start 96.287 112.837) (end 96.287 114.213) (width 0.25) (layer "F.Cu") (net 3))
 (segment (start 96.287 114.213) (end 94 116.5) (width 0.25) (layer "F.Cu") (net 3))
 (segment (start 75.35 116.5) (end 71.45 112.6) (width 0.25) (layer "F.Cu") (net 3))
 (segment (start 71.45 112.6) (end 63.05 112.6) (width 0.25) (layer "F.Cu") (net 3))
 (segment (start 95.2 111.75) (end 96.287 112.837) (width 0.25) (layer "F.Cu") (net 3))
 (segment (start 66.95 96.525) (end 66.95 93.8025) (width 0.25) (layer "F.Cu") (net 9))
 (segment (start 85.927501 112.827501) (end 85.927501 109.749301) (width 0.25) (layer "F.Cu") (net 11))
 (segment (start 85.927501 103.749298) (end 83.076799 106.6) (width 0.25) (layer "F.Cu") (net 11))
 (segment (start 85.95 112.85) (end 85.927501 112.827501) (width 0.25) (layer "F.Cu") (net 11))
 (segment (start 83.076799 106.6) (end 77.8375 106.6) (width 0.25) (layer "F.Cu") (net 11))
 (segment (start 66.9375 98.1875) (end 66.95 98.175) (width 0.25) (layer "F.Cu") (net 10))
 (segment (start 66.9375 101.7125) (end 66.9375 98.1875) (width 0.25) (layer "F.Cu") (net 10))
 (segment (start 90.308099 102.928998) (end 90.308099 104.391901) (width 0.25) (layer "F.Cu") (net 8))
 (segment (start 85.977501 100.087102) (end 87.466203 100.087102) (width 0.25) (layer "F.Cu") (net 8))
 (segment (start 76.925 105.6) (end 77.8375 105.6) (width 0.25) (layer "F.Cu") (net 8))
 (segment (start 90.308099 104.391901) (end 86.425 108.275) (width 0.25) (layer "F.Cu") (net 8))
 (segment (start 76.775 108.275) (end 76.6 108.1) (width 0.25) (layer "F.Cu") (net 8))
 (segment (start 86.583101 99.481502) (end 86.583101 94.692699) (width 0.25) (layer "F.Cu") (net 8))
 (segment (start 76.6 105.925) (end 76.925 105.6) (width 0.25) (layer "F.Cu") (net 8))
 (segment (start 86.425 108.275) (end 76.775 108.275) (width 0.25) (layer "F.Cu") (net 8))
 (segment (start 85.977501 100.087102) (end 86.583101 99.481502) (width 0.25) (layer "F.Cu") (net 8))
 (segment (start 87.466203 100.087102) (end 90.308099 102.928998) (width 0.25) (layer "F.Cu") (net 8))
 (segment (start 76.6 108.1) (end 76.6 105.925) (width 0.25) (layer "F.Cu") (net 8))
 (segment (start 86.583101 94.692699) (end 85.977501 94.087099) (width 0.25) (layer "F.Cu") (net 8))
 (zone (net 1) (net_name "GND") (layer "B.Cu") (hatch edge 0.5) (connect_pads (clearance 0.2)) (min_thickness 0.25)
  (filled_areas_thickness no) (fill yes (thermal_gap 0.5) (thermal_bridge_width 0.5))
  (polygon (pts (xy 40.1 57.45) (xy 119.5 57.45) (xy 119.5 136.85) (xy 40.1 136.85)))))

